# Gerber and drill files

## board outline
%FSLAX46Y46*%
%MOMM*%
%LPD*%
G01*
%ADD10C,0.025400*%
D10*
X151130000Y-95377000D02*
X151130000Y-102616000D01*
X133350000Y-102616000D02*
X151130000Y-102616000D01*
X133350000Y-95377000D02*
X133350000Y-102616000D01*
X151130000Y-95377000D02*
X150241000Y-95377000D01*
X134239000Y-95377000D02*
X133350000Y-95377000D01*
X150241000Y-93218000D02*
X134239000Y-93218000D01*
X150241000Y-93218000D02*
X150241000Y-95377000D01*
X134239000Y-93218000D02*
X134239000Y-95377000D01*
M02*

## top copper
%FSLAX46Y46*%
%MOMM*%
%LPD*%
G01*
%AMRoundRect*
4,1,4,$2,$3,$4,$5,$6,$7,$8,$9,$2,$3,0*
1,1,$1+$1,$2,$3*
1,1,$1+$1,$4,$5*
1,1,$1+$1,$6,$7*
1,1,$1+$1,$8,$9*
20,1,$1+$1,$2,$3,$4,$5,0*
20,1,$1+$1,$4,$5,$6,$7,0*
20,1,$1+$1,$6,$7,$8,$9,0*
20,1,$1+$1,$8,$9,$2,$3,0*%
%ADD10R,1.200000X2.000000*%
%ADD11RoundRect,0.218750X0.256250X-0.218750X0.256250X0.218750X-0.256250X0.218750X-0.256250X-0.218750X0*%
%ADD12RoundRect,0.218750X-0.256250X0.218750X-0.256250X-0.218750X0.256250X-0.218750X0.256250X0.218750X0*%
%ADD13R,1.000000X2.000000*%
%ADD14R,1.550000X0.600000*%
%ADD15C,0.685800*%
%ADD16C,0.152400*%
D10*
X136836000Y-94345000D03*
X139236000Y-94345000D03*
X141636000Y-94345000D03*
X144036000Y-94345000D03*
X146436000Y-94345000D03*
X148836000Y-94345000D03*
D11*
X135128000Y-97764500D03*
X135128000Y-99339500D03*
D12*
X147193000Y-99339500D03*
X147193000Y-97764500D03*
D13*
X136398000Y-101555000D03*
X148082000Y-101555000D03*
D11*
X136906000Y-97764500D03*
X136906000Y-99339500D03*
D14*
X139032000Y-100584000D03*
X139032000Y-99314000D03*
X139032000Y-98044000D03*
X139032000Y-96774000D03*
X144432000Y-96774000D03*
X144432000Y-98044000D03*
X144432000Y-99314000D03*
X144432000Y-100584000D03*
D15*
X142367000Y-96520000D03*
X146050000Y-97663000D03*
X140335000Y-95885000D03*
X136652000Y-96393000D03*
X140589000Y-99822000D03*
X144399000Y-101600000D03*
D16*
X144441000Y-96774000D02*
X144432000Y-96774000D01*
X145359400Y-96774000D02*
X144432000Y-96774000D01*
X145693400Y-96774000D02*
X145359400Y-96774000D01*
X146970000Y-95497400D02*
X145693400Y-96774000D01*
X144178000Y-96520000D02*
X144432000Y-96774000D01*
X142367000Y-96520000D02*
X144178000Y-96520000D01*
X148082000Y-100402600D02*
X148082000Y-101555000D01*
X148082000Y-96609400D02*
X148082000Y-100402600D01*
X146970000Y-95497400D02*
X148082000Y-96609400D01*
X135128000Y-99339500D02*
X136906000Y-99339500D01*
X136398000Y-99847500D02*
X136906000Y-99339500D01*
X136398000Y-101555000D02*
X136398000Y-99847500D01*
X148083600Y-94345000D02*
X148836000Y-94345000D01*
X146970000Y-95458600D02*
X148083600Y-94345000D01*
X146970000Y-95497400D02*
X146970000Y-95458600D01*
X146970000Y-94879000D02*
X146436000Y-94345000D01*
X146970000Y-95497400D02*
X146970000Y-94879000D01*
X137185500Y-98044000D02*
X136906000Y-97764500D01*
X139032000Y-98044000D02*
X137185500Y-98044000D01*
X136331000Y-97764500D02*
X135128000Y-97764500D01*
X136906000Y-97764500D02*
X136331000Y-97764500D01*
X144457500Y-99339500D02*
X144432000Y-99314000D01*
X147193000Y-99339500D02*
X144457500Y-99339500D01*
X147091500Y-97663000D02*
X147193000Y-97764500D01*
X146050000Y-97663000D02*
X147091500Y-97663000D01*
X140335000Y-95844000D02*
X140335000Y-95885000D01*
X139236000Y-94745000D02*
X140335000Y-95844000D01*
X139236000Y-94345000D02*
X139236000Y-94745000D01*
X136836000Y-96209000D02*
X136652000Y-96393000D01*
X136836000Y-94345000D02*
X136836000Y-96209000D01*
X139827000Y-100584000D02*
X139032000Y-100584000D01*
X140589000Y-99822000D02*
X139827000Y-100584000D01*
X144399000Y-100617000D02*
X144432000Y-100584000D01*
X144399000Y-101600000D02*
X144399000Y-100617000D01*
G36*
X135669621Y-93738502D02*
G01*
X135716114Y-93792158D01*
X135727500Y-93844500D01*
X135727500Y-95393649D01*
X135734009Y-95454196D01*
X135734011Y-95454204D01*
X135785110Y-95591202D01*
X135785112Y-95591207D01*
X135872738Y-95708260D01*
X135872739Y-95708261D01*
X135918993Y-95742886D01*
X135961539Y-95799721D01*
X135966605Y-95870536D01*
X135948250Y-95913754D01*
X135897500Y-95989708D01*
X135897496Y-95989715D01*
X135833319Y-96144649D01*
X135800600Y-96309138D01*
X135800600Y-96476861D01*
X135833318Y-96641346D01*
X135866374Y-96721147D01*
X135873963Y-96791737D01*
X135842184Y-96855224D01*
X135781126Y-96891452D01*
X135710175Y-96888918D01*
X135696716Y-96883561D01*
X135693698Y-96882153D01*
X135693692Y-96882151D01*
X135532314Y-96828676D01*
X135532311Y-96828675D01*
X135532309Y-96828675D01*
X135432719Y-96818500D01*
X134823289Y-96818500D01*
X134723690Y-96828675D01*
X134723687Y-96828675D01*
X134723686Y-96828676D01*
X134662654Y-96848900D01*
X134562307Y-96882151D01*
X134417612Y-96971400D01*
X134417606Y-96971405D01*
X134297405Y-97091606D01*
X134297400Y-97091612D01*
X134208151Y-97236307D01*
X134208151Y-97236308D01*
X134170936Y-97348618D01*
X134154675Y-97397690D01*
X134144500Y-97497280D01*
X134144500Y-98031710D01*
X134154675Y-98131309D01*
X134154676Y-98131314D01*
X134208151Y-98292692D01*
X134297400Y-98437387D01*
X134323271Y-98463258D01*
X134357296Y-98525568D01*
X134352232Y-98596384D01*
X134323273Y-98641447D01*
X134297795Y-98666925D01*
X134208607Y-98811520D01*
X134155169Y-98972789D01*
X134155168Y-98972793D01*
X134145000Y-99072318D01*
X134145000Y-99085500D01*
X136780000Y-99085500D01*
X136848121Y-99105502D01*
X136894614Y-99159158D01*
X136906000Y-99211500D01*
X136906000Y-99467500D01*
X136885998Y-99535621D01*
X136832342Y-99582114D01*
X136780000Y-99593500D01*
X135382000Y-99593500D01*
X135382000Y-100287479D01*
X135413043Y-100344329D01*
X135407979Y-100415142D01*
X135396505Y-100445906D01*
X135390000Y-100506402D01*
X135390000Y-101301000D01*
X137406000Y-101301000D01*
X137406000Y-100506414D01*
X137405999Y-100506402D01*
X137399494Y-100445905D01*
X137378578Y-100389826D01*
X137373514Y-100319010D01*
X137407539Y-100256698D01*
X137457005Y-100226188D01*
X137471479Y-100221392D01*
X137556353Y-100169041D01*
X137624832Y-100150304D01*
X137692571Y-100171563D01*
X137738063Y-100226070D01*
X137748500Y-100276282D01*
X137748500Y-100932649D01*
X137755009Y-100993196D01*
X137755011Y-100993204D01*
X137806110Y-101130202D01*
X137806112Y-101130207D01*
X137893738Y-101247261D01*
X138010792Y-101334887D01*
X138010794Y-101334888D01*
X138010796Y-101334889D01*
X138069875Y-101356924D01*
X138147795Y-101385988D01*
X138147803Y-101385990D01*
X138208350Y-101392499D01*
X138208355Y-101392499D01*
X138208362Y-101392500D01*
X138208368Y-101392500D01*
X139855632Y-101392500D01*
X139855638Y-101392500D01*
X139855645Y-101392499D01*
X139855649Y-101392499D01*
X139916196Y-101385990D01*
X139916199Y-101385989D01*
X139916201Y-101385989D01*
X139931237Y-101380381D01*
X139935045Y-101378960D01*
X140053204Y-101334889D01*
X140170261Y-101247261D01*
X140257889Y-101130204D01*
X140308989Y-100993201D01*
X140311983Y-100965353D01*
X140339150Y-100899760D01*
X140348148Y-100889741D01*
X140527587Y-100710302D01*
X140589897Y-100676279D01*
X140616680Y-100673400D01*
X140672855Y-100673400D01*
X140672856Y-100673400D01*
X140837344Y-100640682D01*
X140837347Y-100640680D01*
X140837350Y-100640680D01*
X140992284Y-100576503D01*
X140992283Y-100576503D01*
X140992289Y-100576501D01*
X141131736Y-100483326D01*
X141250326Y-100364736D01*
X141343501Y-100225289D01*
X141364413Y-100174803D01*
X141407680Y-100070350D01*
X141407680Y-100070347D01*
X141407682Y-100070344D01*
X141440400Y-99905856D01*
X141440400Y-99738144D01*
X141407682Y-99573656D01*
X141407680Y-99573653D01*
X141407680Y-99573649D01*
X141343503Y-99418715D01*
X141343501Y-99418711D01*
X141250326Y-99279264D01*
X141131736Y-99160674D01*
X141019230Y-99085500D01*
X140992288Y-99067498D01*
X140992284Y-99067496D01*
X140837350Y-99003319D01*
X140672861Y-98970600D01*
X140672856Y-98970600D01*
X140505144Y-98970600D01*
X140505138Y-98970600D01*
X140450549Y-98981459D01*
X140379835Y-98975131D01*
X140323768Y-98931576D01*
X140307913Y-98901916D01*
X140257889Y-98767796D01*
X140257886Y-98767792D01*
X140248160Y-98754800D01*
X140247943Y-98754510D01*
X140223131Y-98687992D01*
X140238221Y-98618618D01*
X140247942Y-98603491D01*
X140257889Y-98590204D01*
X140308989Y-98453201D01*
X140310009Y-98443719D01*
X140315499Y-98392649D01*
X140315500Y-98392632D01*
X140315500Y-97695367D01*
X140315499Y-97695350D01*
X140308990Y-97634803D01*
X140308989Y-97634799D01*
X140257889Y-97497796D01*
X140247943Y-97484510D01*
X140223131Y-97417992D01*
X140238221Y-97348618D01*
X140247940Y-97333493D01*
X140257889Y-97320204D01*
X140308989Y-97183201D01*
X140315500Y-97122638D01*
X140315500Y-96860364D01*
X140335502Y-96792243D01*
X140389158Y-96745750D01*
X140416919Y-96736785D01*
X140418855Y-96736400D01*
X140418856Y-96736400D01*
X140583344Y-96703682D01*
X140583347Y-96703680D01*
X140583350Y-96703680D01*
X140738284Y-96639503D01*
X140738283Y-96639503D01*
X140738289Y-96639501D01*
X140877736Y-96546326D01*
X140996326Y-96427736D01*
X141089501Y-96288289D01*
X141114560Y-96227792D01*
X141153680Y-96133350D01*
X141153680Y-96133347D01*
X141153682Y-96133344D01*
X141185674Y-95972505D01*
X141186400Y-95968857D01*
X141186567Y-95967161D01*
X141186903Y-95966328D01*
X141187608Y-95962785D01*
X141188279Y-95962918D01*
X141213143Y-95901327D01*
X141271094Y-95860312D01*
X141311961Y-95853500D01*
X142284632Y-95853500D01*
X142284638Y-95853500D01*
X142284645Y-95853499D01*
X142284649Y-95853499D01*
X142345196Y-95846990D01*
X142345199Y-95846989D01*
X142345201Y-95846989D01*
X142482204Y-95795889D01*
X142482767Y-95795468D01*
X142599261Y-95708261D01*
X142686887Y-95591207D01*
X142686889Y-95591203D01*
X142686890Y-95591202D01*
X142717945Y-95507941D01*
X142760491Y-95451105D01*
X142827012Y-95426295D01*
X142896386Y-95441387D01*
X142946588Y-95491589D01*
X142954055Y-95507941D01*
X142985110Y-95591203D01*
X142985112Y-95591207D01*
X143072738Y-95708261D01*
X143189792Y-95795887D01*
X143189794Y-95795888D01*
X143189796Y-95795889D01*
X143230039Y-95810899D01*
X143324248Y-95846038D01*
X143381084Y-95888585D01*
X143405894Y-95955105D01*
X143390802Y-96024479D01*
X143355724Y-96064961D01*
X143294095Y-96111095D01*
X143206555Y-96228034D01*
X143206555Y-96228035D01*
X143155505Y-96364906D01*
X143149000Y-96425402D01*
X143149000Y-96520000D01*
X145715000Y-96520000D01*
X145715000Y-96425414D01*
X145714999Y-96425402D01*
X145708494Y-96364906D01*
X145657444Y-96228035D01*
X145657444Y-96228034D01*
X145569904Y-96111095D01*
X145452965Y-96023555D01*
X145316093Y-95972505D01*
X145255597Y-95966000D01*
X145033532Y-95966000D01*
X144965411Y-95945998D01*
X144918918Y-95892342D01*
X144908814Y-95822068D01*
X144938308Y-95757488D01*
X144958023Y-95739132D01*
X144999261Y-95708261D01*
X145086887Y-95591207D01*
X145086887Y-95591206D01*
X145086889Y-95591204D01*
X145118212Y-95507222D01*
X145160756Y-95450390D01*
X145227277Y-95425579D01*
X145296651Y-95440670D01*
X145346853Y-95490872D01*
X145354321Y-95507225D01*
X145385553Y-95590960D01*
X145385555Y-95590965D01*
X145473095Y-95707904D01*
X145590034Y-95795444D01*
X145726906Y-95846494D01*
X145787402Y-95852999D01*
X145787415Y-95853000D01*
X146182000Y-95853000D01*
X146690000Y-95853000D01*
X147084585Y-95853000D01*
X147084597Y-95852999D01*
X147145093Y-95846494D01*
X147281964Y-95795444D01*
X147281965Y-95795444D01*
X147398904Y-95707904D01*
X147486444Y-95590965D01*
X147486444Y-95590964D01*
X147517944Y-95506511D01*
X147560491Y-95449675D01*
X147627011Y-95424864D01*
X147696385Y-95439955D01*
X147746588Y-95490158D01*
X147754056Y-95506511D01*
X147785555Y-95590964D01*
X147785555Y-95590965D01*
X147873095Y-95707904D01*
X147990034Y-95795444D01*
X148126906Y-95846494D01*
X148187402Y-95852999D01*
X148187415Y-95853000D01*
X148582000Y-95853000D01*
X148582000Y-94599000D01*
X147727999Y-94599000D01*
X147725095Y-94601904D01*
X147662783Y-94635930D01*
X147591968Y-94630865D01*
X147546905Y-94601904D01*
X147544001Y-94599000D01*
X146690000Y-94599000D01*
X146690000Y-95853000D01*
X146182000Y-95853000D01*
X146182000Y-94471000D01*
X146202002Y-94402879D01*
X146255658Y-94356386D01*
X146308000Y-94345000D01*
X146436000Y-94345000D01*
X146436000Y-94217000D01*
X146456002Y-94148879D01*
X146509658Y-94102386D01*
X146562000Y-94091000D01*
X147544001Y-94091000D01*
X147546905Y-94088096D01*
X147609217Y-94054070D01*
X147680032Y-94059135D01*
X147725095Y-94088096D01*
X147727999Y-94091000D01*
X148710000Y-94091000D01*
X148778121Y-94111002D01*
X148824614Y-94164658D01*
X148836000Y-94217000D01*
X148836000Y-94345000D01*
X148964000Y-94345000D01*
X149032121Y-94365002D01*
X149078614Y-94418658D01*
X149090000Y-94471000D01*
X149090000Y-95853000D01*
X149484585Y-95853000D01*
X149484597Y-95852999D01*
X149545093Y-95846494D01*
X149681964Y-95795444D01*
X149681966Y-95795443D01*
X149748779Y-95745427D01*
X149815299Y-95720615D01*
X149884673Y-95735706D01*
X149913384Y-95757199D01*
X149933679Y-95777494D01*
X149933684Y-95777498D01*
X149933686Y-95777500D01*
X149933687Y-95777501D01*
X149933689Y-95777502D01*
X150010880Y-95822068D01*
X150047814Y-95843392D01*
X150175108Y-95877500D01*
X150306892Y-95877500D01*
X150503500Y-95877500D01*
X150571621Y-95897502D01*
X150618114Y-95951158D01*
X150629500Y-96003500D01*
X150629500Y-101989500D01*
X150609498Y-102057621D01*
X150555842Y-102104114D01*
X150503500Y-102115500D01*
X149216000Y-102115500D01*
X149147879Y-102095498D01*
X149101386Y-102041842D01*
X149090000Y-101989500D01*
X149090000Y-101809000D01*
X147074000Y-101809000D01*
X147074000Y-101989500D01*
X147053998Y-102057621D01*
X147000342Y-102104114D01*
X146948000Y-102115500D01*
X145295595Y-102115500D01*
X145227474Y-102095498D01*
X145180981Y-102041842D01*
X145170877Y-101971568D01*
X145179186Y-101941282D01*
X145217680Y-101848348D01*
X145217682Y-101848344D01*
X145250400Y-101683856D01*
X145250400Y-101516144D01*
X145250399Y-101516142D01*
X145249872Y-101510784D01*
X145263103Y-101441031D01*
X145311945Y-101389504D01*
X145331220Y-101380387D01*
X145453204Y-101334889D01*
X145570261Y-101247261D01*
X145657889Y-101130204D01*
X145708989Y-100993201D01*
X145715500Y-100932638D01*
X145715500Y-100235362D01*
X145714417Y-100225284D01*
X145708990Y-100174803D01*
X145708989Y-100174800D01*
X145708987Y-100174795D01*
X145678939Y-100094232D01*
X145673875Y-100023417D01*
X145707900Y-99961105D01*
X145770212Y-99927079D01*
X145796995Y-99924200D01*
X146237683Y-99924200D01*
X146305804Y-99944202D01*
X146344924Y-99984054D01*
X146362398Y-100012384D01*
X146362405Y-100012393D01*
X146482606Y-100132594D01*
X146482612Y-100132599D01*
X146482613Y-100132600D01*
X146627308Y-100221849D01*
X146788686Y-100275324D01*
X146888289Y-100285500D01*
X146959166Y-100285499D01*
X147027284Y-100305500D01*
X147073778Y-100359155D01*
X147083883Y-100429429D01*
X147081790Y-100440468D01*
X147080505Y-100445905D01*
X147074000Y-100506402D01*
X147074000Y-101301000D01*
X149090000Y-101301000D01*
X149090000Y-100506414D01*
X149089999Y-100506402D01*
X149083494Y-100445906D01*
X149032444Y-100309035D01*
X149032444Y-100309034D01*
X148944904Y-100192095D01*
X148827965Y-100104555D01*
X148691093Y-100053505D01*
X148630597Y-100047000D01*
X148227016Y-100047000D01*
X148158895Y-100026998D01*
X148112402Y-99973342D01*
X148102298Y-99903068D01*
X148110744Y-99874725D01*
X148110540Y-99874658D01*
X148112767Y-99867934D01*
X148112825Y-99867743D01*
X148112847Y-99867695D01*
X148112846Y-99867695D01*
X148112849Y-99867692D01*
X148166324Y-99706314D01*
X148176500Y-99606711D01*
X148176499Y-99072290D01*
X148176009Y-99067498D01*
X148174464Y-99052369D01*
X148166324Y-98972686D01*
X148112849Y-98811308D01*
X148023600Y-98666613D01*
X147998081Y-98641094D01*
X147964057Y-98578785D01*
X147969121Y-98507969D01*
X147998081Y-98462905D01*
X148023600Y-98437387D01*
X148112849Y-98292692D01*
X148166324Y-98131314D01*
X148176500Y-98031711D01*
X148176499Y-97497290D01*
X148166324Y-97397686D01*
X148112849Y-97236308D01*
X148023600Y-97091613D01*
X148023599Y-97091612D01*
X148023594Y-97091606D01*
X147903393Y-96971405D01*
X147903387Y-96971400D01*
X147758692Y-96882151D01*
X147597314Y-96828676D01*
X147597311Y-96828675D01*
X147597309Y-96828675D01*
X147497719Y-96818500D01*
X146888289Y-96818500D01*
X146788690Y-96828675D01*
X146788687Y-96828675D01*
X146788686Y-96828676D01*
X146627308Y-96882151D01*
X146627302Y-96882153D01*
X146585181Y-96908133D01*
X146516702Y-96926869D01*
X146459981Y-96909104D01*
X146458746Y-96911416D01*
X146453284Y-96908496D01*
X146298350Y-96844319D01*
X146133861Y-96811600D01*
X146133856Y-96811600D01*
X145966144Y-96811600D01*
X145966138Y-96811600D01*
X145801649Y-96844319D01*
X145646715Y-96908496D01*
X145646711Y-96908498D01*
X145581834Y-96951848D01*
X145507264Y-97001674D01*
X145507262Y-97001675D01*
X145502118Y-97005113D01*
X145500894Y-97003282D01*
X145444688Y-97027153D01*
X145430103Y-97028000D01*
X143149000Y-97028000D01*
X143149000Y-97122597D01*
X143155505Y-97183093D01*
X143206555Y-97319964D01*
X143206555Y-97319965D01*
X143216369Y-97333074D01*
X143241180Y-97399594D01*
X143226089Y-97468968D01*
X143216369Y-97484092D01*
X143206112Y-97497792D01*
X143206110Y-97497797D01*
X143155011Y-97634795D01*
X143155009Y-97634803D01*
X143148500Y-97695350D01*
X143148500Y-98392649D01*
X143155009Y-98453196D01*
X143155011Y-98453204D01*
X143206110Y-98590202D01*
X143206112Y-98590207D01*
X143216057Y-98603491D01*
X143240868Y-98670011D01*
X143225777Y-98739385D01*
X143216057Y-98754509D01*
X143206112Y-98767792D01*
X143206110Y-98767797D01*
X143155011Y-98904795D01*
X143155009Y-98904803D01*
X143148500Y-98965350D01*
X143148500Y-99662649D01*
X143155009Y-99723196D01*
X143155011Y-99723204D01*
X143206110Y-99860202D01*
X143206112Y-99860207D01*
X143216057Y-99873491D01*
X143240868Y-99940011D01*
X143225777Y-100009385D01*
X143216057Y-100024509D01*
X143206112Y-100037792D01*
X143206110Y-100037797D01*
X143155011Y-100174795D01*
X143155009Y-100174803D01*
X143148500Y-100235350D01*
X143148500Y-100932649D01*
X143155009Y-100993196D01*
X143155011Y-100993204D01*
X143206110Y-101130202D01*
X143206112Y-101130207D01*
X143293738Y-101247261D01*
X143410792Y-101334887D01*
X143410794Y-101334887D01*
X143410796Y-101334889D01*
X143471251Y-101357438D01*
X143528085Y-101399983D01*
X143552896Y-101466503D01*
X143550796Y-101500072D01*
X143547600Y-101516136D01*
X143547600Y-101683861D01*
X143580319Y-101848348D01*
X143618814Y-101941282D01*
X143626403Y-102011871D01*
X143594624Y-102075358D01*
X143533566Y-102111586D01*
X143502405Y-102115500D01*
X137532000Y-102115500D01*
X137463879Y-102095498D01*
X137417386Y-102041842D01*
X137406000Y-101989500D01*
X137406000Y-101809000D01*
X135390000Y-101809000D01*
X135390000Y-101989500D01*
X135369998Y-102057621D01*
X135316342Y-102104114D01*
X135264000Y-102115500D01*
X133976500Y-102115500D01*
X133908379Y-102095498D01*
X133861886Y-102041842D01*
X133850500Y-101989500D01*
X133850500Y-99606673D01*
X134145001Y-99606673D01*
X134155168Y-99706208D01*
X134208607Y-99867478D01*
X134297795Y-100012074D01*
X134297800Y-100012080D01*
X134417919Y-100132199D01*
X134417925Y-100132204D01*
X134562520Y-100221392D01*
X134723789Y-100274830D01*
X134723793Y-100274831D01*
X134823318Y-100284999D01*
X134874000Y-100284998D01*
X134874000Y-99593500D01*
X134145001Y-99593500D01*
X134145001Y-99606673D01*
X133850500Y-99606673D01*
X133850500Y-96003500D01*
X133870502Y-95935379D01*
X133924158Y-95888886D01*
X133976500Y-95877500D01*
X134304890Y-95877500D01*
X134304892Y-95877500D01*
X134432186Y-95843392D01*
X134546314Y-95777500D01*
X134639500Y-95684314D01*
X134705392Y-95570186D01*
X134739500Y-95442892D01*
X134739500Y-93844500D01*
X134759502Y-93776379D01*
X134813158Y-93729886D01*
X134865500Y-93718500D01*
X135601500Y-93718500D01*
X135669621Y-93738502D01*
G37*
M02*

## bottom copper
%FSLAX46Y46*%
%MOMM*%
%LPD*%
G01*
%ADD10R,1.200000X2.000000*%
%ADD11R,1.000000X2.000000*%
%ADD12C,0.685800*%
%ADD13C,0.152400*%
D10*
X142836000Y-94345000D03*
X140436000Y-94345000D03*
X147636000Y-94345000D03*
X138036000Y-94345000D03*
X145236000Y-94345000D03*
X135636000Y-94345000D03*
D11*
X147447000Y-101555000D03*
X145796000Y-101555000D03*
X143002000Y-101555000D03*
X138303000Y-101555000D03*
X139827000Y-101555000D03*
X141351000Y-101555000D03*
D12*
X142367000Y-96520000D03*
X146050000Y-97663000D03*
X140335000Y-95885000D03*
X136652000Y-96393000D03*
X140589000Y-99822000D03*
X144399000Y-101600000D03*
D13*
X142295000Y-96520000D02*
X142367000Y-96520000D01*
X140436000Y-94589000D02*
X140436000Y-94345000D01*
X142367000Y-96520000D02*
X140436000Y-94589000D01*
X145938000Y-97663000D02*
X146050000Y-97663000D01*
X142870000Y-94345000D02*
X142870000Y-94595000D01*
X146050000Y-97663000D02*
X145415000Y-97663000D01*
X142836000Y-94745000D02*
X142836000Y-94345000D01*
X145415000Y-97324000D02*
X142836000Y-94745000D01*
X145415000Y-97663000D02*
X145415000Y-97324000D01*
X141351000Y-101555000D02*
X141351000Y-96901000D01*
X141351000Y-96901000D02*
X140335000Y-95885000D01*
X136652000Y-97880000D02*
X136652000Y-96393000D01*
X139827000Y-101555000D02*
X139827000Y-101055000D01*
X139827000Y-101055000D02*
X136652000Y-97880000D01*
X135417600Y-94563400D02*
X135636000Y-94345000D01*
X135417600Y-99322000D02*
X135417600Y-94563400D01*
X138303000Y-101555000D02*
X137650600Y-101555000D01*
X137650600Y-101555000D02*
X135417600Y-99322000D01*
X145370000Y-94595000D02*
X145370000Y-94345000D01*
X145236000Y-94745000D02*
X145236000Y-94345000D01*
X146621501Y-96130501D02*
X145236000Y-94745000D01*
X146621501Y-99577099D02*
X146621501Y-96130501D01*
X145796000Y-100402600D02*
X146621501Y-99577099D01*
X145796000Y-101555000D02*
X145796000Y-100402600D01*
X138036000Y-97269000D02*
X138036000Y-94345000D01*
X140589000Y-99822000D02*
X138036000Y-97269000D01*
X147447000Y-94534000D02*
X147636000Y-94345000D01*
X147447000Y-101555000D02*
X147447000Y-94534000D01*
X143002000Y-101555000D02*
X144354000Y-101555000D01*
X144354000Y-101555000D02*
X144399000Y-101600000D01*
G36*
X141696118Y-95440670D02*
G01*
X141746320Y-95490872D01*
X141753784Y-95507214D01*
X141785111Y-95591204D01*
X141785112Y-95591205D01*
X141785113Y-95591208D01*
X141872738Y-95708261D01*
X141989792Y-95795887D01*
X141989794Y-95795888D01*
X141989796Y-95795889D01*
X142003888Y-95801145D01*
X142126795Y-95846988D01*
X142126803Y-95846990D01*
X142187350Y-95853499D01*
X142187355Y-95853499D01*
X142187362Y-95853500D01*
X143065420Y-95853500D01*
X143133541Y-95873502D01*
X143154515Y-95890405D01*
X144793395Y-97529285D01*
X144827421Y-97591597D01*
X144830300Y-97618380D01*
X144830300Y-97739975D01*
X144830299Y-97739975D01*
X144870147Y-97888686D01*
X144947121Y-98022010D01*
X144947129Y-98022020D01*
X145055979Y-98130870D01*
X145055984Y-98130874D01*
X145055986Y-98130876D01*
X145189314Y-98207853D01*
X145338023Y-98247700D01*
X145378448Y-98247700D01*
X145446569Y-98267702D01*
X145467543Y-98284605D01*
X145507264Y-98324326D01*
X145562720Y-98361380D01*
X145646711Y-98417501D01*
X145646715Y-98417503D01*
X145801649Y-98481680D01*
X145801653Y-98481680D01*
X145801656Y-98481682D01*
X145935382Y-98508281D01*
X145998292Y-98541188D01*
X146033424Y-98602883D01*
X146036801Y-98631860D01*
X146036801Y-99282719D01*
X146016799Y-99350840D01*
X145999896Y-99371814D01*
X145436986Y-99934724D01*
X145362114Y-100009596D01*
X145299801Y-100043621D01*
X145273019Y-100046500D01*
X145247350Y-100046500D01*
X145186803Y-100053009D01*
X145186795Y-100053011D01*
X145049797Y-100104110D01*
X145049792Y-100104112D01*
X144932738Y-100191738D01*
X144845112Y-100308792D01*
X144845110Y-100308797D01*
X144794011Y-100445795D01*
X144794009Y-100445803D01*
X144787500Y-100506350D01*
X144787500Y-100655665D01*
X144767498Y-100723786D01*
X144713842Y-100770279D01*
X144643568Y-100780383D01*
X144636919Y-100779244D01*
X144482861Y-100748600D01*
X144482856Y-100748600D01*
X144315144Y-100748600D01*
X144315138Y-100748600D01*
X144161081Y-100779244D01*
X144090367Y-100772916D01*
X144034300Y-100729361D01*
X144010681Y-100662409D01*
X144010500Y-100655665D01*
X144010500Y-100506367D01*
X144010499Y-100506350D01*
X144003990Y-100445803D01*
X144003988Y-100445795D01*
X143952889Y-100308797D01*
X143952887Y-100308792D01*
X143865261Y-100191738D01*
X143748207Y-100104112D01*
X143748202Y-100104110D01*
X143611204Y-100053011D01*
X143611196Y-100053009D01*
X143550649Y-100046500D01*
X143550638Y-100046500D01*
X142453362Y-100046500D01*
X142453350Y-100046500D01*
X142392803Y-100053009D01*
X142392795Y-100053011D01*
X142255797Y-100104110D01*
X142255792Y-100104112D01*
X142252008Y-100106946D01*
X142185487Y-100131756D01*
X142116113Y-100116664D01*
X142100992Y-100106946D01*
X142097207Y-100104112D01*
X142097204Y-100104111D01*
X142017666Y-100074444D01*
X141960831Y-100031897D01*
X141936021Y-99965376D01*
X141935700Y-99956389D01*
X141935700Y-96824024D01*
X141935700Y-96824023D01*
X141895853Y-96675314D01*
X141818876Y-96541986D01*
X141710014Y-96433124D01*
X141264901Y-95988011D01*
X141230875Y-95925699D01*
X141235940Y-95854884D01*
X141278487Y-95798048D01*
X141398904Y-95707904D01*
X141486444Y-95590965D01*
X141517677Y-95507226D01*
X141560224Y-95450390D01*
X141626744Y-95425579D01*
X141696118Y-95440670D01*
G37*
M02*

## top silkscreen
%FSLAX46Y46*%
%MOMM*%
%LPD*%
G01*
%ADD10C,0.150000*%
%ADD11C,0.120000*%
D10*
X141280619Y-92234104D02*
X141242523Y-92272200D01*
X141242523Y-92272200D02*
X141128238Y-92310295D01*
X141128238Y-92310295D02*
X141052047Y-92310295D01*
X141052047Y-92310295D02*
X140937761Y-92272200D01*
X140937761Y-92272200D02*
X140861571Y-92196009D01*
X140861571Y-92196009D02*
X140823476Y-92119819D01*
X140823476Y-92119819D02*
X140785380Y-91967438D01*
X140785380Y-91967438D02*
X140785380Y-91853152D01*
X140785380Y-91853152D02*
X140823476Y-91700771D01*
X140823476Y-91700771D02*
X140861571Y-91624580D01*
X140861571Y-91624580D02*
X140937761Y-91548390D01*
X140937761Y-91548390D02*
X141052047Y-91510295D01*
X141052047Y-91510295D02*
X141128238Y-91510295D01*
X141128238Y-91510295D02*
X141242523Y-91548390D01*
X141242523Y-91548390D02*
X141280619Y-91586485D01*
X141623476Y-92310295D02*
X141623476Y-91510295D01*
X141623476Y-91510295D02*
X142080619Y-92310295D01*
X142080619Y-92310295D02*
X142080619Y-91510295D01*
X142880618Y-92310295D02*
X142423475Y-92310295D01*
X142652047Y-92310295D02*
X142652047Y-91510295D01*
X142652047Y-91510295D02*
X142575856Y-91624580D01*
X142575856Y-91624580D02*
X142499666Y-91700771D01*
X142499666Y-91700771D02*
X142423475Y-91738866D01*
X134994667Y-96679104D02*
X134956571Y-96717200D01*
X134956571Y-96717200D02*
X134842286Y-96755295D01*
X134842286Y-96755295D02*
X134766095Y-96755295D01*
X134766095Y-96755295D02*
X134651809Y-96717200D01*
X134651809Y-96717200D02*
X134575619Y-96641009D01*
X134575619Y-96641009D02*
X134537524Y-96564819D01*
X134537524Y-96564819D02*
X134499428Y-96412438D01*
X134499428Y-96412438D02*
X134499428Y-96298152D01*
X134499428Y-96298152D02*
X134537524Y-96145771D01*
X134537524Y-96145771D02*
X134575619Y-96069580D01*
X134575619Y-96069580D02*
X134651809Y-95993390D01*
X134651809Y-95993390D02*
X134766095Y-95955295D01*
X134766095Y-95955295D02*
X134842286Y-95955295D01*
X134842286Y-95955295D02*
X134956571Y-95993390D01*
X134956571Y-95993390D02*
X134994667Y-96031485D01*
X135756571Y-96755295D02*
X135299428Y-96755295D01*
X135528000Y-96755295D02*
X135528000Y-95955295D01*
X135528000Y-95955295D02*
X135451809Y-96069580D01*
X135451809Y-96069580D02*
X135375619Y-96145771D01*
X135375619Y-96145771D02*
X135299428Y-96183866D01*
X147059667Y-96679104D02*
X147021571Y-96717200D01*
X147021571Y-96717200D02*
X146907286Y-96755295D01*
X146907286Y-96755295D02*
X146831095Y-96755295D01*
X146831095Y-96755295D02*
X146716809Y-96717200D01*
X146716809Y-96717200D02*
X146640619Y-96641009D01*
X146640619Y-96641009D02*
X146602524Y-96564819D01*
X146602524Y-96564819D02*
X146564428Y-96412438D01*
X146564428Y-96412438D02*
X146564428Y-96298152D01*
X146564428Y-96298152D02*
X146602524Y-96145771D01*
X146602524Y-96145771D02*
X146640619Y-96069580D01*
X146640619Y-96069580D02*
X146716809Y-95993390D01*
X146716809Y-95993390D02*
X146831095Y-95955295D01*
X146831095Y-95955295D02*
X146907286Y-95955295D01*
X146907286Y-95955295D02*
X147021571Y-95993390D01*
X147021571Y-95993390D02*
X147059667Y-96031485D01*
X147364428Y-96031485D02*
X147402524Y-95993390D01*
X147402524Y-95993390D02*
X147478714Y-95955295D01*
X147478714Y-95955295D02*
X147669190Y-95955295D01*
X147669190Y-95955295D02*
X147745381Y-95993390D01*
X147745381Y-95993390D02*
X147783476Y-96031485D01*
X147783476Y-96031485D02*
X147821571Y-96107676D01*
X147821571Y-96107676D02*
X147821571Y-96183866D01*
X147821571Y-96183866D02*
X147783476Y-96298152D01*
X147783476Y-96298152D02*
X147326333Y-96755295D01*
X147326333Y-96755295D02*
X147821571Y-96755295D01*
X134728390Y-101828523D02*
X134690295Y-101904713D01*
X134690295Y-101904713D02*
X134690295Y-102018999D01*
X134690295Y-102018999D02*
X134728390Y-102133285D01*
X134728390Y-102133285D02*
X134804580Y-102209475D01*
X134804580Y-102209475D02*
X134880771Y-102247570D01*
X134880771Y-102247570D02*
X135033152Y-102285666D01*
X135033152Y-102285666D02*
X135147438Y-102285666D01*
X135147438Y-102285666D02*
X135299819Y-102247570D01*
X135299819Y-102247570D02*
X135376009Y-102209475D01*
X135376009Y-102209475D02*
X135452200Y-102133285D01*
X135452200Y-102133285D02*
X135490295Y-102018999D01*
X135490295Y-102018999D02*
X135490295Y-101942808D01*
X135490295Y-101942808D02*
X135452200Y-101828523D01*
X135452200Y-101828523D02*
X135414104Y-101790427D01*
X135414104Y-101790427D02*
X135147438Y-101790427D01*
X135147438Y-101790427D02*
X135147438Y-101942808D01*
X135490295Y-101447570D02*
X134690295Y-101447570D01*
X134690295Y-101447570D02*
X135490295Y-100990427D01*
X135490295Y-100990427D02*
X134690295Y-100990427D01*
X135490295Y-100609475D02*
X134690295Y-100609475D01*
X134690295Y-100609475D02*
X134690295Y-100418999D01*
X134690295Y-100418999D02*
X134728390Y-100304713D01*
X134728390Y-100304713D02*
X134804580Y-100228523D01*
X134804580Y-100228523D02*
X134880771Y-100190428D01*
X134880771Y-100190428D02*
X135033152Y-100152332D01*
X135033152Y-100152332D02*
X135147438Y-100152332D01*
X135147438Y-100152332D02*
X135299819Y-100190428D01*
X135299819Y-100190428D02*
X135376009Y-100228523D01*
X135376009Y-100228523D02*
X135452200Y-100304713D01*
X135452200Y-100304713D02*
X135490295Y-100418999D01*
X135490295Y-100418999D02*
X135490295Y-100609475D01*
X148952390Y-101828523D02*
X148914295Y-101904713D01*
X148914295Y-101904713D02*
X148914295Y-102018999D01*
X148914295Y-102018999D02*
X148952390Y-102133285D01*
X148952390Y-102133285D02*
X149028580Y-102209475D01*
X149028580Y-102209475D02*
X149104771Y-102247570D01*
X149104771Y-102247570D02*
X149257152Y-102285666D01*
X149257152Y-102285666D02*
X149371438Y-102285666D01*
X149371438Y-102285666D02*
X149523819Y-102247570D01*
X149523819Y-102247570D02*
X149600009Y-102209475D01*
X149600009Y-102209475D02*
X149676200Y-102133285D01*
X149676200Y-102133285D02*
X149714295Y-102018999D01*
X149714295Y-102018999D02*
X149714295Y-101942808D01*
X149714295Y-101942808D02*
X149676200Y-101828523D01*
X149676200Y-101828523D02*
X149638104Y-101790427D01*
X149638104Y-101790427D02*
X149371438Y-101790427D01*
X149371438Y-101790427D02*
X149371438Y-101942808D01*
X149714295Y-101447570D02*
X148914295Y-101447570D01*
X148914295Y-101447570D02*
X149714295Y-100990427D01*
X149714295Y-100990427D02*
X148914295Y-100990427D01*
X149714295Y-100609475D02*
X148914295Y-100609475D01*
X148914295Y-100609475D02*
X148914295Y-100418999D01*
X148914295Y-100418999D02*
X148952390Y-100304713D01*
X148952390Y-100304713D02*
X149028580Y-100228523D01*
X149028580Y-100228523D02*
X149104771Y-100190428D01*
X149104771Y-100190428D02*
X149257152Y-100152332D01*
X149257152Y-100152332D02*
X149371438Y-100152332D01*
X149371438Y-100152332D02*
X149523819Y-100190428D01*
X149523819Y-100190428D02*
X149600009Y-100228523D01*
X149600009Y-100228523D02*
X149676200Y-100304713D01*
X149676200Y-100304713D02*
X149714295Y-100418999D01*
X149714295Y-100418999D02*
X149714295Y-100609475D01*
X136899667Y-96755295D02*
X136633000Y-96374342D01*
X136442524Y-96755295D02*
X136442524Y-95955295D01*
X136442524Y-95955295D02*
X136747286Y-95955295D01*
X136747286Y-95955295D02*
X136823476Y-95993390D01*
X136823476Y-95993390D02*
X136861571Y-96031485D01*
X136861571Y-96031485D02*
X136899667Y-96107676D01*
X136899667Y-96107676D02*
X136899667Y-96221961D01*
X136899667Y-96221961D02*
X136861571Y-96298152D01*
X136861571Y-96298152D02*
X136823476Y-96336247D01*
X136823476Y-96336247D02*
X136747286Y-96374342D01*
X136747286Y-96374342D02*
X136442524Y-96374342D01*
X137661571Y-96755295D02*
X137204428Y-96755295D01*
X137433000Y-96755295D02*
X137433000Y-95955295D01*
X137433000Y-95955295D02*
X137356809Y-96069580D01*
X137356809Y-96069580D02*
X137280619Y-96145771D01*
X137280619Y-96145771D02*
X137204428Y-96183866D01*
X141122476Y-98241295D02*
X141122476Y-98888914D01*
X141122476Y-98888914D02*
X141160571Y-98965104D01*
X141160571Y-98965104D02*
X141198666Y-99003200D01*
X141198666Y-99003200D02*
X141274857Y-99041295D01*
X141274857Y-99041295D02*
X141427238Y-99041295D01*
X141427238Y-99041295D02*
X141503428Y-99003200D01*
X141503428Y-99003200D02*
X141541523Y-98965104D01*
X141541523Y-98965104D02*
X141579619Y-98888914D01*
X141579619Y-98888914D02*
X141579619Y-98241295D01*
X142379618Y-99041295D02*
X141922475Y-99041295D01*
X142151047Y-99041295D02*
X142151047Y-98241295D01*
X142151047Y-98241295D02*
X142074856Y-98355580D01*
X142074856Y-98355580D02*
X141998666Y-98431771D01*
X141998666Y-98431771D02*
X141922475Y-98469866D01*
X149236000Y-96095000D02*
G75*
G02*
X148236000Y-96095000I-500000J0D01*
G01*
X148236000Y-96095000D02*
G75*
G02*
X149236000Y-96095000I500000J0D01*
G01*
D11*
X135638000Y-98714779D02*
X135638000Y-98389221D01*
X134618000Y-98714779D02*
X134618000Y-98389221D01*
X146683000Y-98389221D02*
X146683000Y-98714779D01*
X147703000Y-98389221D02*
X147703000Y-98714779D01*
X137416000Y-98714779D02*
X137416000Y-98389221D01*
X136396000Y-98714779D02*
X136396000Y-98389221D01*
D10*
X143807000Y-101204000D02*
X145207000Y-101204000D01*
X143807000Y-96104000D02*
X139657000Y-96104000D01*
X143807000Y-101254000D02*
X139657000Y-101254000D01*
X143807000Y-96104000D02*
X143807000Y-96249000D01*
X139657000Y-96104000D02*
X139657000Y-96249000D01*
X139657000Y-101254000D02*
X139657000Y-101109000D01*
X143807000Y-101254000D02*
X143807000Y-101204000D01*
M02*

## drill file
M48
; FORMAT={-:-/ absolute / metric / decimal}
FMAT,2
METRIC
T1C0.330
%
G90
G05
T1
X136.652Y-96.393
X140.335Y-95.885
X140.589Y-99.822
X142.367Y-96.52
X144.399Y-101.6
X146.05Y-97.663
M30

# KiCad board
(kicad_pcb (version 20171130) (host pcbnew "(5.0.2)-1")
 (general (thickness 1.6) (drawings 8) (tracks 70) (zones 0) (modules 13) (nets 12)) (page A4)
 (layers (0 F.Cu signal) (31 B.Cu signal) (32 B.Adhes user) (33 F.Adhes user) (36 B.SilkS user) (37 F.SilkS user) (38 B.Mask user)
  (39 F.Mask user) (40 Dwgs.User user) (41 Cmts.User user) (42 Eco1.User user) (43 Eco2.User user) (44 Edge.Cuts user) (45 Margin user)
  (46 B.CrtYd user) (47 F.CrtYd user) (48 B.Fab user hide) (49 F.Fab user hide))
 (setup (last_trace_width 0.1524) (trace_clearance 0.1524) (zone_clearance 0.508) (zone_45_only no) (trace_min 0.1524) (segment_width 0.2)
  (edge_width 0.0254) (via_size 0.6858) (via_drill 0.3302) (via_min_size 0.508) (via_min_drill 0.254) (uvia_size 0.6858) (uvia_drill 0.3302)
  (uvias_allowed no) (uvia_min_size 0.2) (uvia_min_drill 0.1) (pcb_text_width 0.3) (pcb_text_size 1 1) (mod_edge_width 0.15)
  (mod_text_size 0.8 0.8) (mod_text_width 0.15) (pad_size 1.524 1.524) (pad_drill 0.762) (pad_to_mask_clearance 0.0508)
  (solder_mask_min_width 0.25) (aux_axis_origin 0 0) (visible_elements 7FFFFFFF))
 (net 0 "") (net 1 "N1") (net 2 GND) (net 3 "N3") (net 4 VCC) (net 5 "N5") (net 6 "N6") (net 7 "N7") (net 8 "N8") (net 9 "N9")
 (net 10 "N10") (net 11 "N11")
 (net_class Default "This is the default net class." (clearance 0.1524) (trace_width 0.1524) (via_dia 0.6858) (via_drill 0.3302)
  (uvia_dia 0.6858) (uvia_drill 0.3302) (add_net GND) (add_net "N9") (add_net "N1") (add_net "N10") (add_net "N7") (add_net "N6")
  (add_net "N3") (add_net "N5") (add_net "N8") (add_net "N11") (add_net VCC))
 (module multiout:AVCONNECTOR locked (layer F.Cu) (at 141.836 94.345)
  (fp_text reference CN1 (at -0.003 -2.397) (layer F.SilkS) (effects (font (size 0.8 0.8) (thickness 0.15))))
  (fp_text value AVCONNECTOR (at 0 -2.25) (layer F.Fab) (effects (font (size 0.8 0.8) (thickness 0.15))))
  (fp_circle (center 6.9 1.75) (end 7.4 1.75) (layer F.SilkS) (width 0.15))
  (pad 6 connect rect (at 1 0) (size 1.2 2) (layers B.Cu B.Mask) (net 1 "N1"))
  (pad 8 connect rect (at -1.4 0) (size 1.2 2) (layers B.Cu B.Mask) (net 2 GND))
  (pad 2 connect rect (at 5.8 0) (size 1.2 2) (layers B.Cu B.Mask) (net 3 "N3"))
  (pad 10 connect rect (at -3.8 0) (size 1.2 2) (layers B.Cu B.Mask) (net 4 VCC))
  (pad 4 connect rect (at 3.4 0) (size 1.2 2) (layers B.Cu B.Mask) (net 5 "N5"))
  (pad 12 connect rect (at -6.2 0) (size 1.2 2) (layers B.Cu B.Mask) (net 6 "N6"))
  (pad 11 connect rect (at -5 0) (size 1.2 2) (layers F.Cu F.Mask) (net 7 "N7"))
  (pad 9 connect rect (at -2.6 0) (size 1.2 2) (layers F.Cu F.Mask) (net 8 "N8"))
  (pad 7 connect rect (at -0.2 0) (size 1.2 2) (layers F.Cu F.Mask))
  (pad 5 connect rect (at 2.2 0) (size 1.2 2) (layers F.Cu F.Mask))
  (pad 3 connect rect (at 4.6 0) (size 1.2 2) (layers F.Cu F.Mask) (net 2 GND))
  (pad 1 connect rect (at 7 0) (size 1.2 2) (layers F.Cu F.Mask) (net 2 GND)))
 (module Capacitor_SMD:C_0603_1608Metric (layer F.Cu) (at 135.128 98.552 90)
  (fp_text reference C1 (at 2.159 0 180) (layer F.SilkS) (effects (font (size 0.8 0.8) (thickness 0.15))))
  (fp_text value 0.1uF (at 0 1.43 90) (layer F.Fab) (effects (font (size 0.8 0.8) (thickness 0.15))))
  (fp_line (start -0.162779 0.51) (end 0.162779 0.51) (layer F.SilkS) (width 0.12))
  (fp_line (start -0.162779 -0.51) (end 0.162779 -0.51) (layer F.SilkS) (width 0.12))
  (pad 2 smd roundrect (at 0.7875 0 90) (size 0.875 0.95) (layers F.Cu F.Paste F.Mask) (roundrect_rratio 0.25) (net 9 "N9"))
  (pad 1 smd roundrect (at -0.7875 0 90) (size 0.875 0.95) (layers F.Cu F.Paste F.Mask) (roundrect_rratio 0.25) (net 2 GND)))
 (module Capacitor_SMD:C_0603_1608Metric (layer F.Cu) (at 147.193 98.552 270)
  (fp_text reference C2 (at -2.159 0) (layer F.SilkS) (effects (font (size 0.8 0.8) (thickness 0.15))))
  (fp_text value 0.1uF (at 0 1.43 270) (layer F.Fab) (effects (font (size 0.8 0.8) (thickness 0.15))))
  (fp_line (start -0.162779 0.51) (end 0.162779 0.51) (layer F.SilkS) (width 0.12))
  (fp_line (start -0.162779 -0.51) (end 0.162779 -0.51) (layer F.SilkS) (width 0.12))
  (pad 2 smd roundrect (at 0.7875 0 270) (size 0.875 0.95) (layers F.Cu F.Paste F.Mask) (roundrect_rratio 0.25) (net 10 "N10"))
  (pad 1 smd roundrect (at -0.7875 0 270) (size 0.875 0.95) (layers F.Cu F.Paste F.Mask) (roundrect_rratio 0.25) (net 1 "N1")))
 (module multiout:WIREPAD (layer B.Cu) (at 147.447 101.555)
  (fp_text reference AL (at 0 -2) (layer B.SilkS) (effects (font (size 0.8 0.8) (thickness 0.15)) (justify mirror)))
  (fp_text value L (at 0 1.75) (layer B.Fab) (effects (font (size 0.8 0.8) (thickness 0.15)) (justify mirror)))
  (pad 1 connect rect (at 0 0) (size 1 2) (layers B.Cu B.Mask) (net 3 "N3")))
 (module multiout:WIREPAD (layer B.Cu) (at 145.796 101.555)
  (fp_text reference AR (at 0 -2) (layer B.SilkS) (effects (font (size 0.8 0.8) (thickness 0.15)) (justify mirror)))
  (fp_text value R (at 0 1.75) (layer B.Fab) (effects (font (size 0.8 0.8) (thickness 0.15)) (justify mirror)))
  (pad 1 connect rect (at 0 0) (size 1 2) (layers B.Cu B.Mask) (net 5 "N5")))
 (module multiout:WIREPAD (layer B.Cu) (at 143.002 101.555)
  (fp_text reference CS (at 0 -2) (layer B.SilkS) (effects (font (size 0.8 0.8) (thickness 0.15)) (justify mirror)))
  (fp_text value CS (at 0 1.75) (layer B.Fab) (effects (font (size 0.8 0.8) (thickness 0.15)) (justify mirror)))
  (pad 1 connect rect (at 0 0) (size 1 2) (layers B.Cu B.Mask) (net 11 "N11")))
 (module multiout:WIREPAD (layer B.Cu) (at 138.303 101.555)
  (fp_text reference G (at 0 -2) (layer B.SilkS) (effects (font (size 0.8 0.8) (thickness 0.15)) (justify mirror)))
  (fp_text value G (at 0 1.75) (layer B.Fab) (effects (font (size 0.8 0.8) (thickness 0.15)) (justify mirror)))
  (pad 1 connect rect (at 0 0) (size 1 2) (layers B.Cu B.Mask) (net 6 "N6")))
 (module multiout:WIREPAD (layer B.Cu) (at 139.827 101.555)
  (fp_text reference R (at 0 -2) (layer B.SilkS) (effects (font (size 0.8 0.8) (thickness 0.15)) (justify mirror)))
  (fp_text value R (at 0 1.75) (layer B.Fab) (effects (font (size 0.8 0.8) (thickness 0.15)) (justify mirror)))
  (pad 1 connect rect (at 0 0) (size 1 2) (layers B.Cu B.Mask) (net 7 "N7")))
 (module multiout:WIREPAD (layer B.Cu) (at 141.351 101.555)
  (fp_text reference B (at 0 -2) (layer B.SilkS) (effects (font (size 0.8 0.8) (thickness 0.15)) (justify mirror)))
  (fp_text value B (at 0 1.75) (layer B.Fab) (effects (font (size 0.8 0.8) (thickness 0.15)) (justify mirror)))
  (pad 1 connect rect (at 0 0) (size 1 2) (layers B.Cu B.Mask) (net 8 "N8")))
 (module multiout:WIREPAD (layer F.Cu) (at 136.398 101.555)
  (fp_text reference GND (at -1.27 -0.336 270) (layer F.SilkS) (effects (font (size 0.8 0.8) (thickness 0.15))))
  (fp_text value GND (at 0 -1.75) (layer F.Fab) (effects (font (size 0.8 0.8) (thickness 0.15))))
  (pad 1 connect rect (at 0 0) (size 1 2) (layers F.Cu F.Mask) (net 2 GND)))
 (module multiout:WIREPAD (layer F.Cu) (at 148.082 101.555)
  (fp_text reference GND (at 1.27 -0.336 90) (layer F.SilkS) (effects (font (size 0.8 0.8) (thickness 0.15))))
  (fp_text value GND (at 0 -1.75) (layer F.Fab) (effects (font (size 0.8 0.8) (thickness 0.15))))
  (pad 1 connect rect (at 0 0) (size 1 2) (layers F.Cu F.Mask) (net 2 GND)))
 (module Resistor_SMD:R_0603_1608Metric (layer F.Cu) (at 136.906 98.552 90)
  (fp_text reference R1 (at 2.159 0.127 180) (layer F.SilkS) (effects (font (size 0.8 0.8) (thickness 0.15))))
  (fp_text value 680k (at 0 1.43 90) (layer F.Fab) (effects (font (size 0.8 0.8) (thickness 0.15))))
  (fp_line (start -0.162779 0.51) (end 0.162779 0.51) (layer F.SilkS) (width 0.12))
  (fp_line (start -0.162779 -0.51) (end 0.162779 -0.51) (layer F.SilkS) (width 0.12))
  (pad 2 smd roundrect (at 0.7875 0 90) (size 0.875 0.95) (layers F.Cu F.Paste F.Mask) (roundrect_rratio 0.25) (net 9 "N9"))
  (pad 1 smd roundrect (at -0.7875 0 90) (size 0.875 0.95) (layers F.Cu F.Paste F.Mask) (roundrect_rratio 0.25) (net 2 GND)))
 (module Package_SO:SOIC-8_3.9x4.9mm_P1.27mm (layer F.Cu) (at 141.732 98.679 180)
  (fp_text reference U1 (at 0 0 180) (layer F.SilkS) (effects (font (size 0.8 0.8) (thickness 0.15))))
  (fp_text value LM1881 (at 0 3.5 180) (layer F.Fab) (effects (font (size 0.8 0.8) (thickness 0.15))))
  (fp_line (start -2.075 -2.525) (end -3.475 -2.525) (layer F.SilkS) (width 0.15))
  (fp_line (start -2.075 2.575) (end 2.075 2.575) (layer F.SilkS) (width 0.15))
  (fp_line (start -2.075 -2.575) (end 2.075 -2.575) (layer F.SilkS) (width 0.15))
  (fp_line (start -2.075 2.575) (end -2.075 2.43) (layer F.SilkS) (width 0.15))
  (fp_line (start 2.075 2.575) (end 2.075 2.43) (layer F.SilkS) (width 0.15))
  (fp_line (start 2.075 -2.575) (end 2.075 -2.43) (layer F.SilkS) (width 0.15))
  (fp_line (start -2.075 -2.575) (end -2.075 -2.525) (layer F.SilkS) (width 0.15))
  (pad 8 smd rect (at 2.7 -1.905 180) (size 1.55 0.6) (layers F.Cu F.Paste F.Mask) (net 4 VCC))
  (pad 7 smd rect (at 2.7 -0.635 180) (size 1.55 0.6) (layers F.Cu F.Paste F.Mask))
  (pad 6 smd rect (at 2.7 0.635 180) (size 1.55 0.6) (layers F.Cu F.Paste F.Mask) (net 9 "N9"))
  (pad 5 smd rect (at 2.7 1.905 180) (size 1.55 0.6) (layers F.Cu F.Paste F.Mask))
  (pad 4 smd rect (at -2.7 1.905 180) (size 1.55 0.6) (layers F.Cu F.Paste F.Mask) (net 2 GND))
  (pad 3 smd rect (at -2.7 0.635 180) (size 1.55 0.6) (layers F.Cu F.Paste F.Mask))
  (pad 2 smd rect (at -2.7 -0.635 180) (size 1.55 0.6) (layers F.Cu F.Paste F.Mask) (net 10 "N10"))
  (pad 1 smd rect (at -2.7 -1.905 180) (size 1.55 0.6) (layers F.Cu F.Paste F.Mask) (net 11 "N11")))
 (gr_line (start 151.13 95.377) (end 151.13 102.616) (layer Edge.Cuts) (width 0.0254))
 (gr_line (start 133.35 102.616) (end 151.13 102.616) (layer Edge.Cuts) (width 0.0254))
 (gr_line (start 133.35 95.377) (end 133.35 102.616) (layer Edge.Cuts) (width 0.0254))
 (gr_line (start 151.13 95.377) (end 150.241 95.377) (layer Edge.Cuts) (width 0.0254))
 (gr_line (start 134.239 95.377) (end 133.35 95.377) (layer Edge.Cuts) (width 0.0254))
 (gr_line (start 150.241 93.218) (end 134.239 93.218) (layer Edge.Cuts) (width 0.0254))
 (gr_line (start 150.241 93.218) (end 150.241 95.377) (layer Edge.Cuts) (width 0.0254))
 (gr_line (start 134.239 93.218) (end 134.239 95.377) (layer Edge.Cuts) (width 0.0254))
 (segment (start 144.441 96.774) (end 144.432 96.774) (width 0.1524) (layer F.Cu) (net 2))
 (via (at 142.367 96.52) (size 0.6858) (drill 0.3302) (layers F.Cu B.Cu) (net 2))
 (segment (start 142.295 96.52) (end 142.367 96.52) (width 0.1524) (layer B.Cu) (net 2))
 (segment (start 145.3594 96.774) (end 144.432 96.774) (width 0.1524) (layer F.Cu) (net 2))
 (segment (start 145.6934 96.774) (end 145.3594 96.774) (width 0.1524) (layer F.Cu) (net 2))
 (segment (start 146.97 95.4974) (end 145.6934 96.774) (width 0.1524) (layer F.Cu) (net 2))
 (segment (start 144.178 96.52) (end 144.432 96.774) (width 0.1524) (layer F.Cu) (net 2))
 (segment (start 142.367 96.52) (end 144.178 96.52) (width 0.1524) (layer F.Cu) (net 2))
 (segment (start 148.082 100.4026) (end 148.082 101.555) (width 0.1524) (layer F.Cu) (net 2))
 (segment (start 148.082 96.6094) (end 148.082 100.4026) (width 0.1524) (layer F.Cu) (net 2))
 (segment (start 146.97 95.4974) (end 148.082 96.6094) (width 0.1524) (layer F.Cu) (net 2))
 (segment (start 135.128 99.3395) (end 136.906 99.3395) (width 0.1524) (layer F.Cu) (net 2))
 (segment (start 136.398 99.8475) (end 136.906 99.3395) (width 0.1524) (layer F.Cu) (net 2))
 (segment (start 136.398 101.555) (end 136.398 99.8475) (width 0.1524) (layer F.Cu) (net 2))
 (segment (start 140.436 94.589) (end 140.436 94.345) (width 0.1524) (layer B.Cu) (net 2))
 (segment (start 142.367 96.52) (end 140.436 94.589) (width 0.1524) (layer B.Cu) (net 2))
 (segment (start 148.0836 94.345) (end 148.836 94.345) (width 0.1524) (layer F.Cu) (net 2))
 (segment (start 146.97 95.4586) (end 148.0836 94.345) (width 0.1524) (layer F.Cu) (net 2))
 (segment (start 146.97 95.4974) (end 146.97 95.4586) (width 0.1524) (layer F.Cu) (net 2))
 (segment (start 146.97 94.879) (end 146.436 94.345) (width 0.1524) (layer F.Cu) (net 2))
 (segment (start 146.97 95.4974) (end 146.97 94.879) (width 0.1524) (layer F.Cu) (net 2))
 (segment (start 137.1855 98.044) (end 136.906 97.7645) (width 0.1524) (layer F.Cu) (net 9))
 (segment (start 139.032 98.044) (end 137.1855 98.044) (width 0.1524) (layer F.Cu) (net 9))
 (segment (start 136.331 97.7645) (end 135.128 97.7645) (width 0.1524) (layer F.Cu) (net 9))
 (segment (start 136.906 97.7645) (end 136.331 97.7645) (width 0.1524) (layer F.Cu) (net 9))
 (segment (start 144.4575 99.3395) (end 144.432 99.314) (width 0.1524) (layer F.Cu) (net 10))
 (segment (start 147.193 99.3395) (end 144.4575 99.3395) (width 0.1524) (layer F.Cu) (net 10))
 (via (at 146.05 97.663) (size 0.6858) (drill 0.3302) (layers F.Cu B.Cu) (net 1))
 (segment (start 145.938 97.663) (end 146.05 97.663) (width 0.1524) (layer B.Cu) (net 1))
 (segment (start 142.87 94.345) (end 142.87 94.595) (width 0.1524) (layer B.Cu) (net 1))
 (segment (start 147.0915 97.663) (end 147.193 97.7645) (width 0.1524) (layer F.Cu) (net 1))
 (segment (start 146.05 97.663) (end 147.0915 97.663) (width 0.1524) (layer F.Cu) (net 1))
 (segment (start 146.05 97.663) (end 145.415 97.663) (width 0.1524) (layer B.Cu) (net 1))
 (segment (start 142.836 94.745) (end 142.836 94.345) (width 0.1524) (layer B.Cu) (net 1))
 (segment (start 145.415 97.324) (end 142.836 94.745) (width 0.1524) (layer B.Cu) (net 1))
 (segment (start 145.415 97.663) (end 145.415 97.324) (width 0.1524) (layer B.Cu) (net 1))
 (via (at 140.335 95.885) (size 0.6858) (drill 0.3302) (layers F.Cu B.Cu) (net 8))
 (segment (start 141.351 101.555) (end 141.351 96.901) (width 0.1524) (layer B.Cu) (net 8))
 (segment (start 141.351 96.901) (end 140.335 95.885) (width 0.1524) (layer B.Cu) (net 8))
 (segment (start 140.335 95.844) (end 140.335 95.885) (width 0.1524) (layer F.Cu) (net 8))
 (segment (start 139.236 94.745) (end 140.335 95.844) (width 0.1524) (layer F.Cu) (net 8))
 (segment (start 139.236 94.345) (end 139.236 94.745) (width 0.1524) (layer F.Cu) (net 8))
 (via (at 136.652 96.393) (size 0.6858) (drill 0.3302) (layers F.Cu B.Cu) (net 7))
 (segment (start 136.652 97.88) (end 136.652 96.393) (width 0.1524) (layer B.Cu) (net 7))
 (segment (start 139.827 101.555) (end 139.827 101.055) (width 0.1524) (layer B.Cu) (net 7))
 (segment (start 139.827 101.055) (end 136.652 97.88) (width 0.1524) (layer B.Cu) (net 7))
 (segment (start 136.836 96.209) (end 136.652 96.393) (width 0.1524) (layer F.Cu) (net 7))
 (segment (start 136.836 94.345) (end 136.836 96.209) (width 0.1524) (layer F.Cu) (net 7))
 (segment (start 135.4176 94.5634) (end 135.636 94.345) (width 0.1524) (layer B.Cu) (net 6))
 (segment (start 135.4176 99.322) (end 135.4176 94.5634) (width 0.1524) (layer B.Cu) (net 6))
 (segment (start 138.303 101.555) (end 137.6506 101.555) (width 0.1524) (layer B.Cu) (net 6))
 (segment (start 137.6506 101.555) (end 135.4176 99.322) (width 0.1524) (layer B.Cu) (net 6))
 (segment (start 145.37 94.595) (end 145.37 94.345) (width 0.1524) (layer B.Cu) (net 5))
 (segment (start 145.236 94.745) (end 145.236 94.345) (width 0.1524) (layer B.Cu) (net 5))
 (segment (start 146.621501 96.130501) (end 145.236 94.745) (width 0.1524) (layer B.Cu) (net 5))
 (segment (start 146.621501 99.577099) (end 146.621501 96.130501) (width 0.1524) (layer B.Cu) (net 5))
 (segment (start 145.796 100.4026) (end 146.621501 99.577099) (width 0.1524) (layer B.Cu) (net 5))
 (segment (start 145.796 101.555) (end 145.796 100.4026) (width 0.1524) (layer B.Cu) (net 5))
 (via (at 140.589 99.822) (size 0.6858) (drill 0.3302) (layers F.Cu B.Cu) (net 4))
 (segment (start 139.827 100.584) (end 139.032 100.584) (width 0.1524) (layer F.Cu) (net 4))
 (segment (start 140.589 99.822) (end 139.827 100.584) (width 0.1524) (layer F.Cu) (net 4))
 (segment (start 138.036 97.269) (end 138.036 94.345) (width 0.1524) (layer B.Cu) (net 4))
 (segment (start 140.589 99.822) (end 138.036 97.269) (width 0.1524) (layer B.Cu) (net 4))
 (segment (start 147.447 94.534) (end 147.636 94.345) (width 0.1524) (layer B.Cu) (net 3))
 (segment (start 147.447 101.555) (end 147.447 94.534) (width 0.1524) (layer B.Cu) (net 3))
 (via (at 144.399 101.6) (size 0.6858) (drill 0.3302) (layers F.Cu B.Cu) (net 11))
 (segment (start 143.002 101.555) (end 144.354 101.555) (width 0.1524) (layer B.Cu) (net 11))
 (segment (start 144.354 101.555) (end 144.399 101.6) (width 0.1524) (layer B.Cu) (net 11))
 (segment (start 144.399 100.617) (end 144.432 100.584) (width 0.1524) (layer F.Cu) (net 11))
 (segment (start 144.399 101.6) (end 144.399 100.617) (width 0.1524) (layer F.Cu) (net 11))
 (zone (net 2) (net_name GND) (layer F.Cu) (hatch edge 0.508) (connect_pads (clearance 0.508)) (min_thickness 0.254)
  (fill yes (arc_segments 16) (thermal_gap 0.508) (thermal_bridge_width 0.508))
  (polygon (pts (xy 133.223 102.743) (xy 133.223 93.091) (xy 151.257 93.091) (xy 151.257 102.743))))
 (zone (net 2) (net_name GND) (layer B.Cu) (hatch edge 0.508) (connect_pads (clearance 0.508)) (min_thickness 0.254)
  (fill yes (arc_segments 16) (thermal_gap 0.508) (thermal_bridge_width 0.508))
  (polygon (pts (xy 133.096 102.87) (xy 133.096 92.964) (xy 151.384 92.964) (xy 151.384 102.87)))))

